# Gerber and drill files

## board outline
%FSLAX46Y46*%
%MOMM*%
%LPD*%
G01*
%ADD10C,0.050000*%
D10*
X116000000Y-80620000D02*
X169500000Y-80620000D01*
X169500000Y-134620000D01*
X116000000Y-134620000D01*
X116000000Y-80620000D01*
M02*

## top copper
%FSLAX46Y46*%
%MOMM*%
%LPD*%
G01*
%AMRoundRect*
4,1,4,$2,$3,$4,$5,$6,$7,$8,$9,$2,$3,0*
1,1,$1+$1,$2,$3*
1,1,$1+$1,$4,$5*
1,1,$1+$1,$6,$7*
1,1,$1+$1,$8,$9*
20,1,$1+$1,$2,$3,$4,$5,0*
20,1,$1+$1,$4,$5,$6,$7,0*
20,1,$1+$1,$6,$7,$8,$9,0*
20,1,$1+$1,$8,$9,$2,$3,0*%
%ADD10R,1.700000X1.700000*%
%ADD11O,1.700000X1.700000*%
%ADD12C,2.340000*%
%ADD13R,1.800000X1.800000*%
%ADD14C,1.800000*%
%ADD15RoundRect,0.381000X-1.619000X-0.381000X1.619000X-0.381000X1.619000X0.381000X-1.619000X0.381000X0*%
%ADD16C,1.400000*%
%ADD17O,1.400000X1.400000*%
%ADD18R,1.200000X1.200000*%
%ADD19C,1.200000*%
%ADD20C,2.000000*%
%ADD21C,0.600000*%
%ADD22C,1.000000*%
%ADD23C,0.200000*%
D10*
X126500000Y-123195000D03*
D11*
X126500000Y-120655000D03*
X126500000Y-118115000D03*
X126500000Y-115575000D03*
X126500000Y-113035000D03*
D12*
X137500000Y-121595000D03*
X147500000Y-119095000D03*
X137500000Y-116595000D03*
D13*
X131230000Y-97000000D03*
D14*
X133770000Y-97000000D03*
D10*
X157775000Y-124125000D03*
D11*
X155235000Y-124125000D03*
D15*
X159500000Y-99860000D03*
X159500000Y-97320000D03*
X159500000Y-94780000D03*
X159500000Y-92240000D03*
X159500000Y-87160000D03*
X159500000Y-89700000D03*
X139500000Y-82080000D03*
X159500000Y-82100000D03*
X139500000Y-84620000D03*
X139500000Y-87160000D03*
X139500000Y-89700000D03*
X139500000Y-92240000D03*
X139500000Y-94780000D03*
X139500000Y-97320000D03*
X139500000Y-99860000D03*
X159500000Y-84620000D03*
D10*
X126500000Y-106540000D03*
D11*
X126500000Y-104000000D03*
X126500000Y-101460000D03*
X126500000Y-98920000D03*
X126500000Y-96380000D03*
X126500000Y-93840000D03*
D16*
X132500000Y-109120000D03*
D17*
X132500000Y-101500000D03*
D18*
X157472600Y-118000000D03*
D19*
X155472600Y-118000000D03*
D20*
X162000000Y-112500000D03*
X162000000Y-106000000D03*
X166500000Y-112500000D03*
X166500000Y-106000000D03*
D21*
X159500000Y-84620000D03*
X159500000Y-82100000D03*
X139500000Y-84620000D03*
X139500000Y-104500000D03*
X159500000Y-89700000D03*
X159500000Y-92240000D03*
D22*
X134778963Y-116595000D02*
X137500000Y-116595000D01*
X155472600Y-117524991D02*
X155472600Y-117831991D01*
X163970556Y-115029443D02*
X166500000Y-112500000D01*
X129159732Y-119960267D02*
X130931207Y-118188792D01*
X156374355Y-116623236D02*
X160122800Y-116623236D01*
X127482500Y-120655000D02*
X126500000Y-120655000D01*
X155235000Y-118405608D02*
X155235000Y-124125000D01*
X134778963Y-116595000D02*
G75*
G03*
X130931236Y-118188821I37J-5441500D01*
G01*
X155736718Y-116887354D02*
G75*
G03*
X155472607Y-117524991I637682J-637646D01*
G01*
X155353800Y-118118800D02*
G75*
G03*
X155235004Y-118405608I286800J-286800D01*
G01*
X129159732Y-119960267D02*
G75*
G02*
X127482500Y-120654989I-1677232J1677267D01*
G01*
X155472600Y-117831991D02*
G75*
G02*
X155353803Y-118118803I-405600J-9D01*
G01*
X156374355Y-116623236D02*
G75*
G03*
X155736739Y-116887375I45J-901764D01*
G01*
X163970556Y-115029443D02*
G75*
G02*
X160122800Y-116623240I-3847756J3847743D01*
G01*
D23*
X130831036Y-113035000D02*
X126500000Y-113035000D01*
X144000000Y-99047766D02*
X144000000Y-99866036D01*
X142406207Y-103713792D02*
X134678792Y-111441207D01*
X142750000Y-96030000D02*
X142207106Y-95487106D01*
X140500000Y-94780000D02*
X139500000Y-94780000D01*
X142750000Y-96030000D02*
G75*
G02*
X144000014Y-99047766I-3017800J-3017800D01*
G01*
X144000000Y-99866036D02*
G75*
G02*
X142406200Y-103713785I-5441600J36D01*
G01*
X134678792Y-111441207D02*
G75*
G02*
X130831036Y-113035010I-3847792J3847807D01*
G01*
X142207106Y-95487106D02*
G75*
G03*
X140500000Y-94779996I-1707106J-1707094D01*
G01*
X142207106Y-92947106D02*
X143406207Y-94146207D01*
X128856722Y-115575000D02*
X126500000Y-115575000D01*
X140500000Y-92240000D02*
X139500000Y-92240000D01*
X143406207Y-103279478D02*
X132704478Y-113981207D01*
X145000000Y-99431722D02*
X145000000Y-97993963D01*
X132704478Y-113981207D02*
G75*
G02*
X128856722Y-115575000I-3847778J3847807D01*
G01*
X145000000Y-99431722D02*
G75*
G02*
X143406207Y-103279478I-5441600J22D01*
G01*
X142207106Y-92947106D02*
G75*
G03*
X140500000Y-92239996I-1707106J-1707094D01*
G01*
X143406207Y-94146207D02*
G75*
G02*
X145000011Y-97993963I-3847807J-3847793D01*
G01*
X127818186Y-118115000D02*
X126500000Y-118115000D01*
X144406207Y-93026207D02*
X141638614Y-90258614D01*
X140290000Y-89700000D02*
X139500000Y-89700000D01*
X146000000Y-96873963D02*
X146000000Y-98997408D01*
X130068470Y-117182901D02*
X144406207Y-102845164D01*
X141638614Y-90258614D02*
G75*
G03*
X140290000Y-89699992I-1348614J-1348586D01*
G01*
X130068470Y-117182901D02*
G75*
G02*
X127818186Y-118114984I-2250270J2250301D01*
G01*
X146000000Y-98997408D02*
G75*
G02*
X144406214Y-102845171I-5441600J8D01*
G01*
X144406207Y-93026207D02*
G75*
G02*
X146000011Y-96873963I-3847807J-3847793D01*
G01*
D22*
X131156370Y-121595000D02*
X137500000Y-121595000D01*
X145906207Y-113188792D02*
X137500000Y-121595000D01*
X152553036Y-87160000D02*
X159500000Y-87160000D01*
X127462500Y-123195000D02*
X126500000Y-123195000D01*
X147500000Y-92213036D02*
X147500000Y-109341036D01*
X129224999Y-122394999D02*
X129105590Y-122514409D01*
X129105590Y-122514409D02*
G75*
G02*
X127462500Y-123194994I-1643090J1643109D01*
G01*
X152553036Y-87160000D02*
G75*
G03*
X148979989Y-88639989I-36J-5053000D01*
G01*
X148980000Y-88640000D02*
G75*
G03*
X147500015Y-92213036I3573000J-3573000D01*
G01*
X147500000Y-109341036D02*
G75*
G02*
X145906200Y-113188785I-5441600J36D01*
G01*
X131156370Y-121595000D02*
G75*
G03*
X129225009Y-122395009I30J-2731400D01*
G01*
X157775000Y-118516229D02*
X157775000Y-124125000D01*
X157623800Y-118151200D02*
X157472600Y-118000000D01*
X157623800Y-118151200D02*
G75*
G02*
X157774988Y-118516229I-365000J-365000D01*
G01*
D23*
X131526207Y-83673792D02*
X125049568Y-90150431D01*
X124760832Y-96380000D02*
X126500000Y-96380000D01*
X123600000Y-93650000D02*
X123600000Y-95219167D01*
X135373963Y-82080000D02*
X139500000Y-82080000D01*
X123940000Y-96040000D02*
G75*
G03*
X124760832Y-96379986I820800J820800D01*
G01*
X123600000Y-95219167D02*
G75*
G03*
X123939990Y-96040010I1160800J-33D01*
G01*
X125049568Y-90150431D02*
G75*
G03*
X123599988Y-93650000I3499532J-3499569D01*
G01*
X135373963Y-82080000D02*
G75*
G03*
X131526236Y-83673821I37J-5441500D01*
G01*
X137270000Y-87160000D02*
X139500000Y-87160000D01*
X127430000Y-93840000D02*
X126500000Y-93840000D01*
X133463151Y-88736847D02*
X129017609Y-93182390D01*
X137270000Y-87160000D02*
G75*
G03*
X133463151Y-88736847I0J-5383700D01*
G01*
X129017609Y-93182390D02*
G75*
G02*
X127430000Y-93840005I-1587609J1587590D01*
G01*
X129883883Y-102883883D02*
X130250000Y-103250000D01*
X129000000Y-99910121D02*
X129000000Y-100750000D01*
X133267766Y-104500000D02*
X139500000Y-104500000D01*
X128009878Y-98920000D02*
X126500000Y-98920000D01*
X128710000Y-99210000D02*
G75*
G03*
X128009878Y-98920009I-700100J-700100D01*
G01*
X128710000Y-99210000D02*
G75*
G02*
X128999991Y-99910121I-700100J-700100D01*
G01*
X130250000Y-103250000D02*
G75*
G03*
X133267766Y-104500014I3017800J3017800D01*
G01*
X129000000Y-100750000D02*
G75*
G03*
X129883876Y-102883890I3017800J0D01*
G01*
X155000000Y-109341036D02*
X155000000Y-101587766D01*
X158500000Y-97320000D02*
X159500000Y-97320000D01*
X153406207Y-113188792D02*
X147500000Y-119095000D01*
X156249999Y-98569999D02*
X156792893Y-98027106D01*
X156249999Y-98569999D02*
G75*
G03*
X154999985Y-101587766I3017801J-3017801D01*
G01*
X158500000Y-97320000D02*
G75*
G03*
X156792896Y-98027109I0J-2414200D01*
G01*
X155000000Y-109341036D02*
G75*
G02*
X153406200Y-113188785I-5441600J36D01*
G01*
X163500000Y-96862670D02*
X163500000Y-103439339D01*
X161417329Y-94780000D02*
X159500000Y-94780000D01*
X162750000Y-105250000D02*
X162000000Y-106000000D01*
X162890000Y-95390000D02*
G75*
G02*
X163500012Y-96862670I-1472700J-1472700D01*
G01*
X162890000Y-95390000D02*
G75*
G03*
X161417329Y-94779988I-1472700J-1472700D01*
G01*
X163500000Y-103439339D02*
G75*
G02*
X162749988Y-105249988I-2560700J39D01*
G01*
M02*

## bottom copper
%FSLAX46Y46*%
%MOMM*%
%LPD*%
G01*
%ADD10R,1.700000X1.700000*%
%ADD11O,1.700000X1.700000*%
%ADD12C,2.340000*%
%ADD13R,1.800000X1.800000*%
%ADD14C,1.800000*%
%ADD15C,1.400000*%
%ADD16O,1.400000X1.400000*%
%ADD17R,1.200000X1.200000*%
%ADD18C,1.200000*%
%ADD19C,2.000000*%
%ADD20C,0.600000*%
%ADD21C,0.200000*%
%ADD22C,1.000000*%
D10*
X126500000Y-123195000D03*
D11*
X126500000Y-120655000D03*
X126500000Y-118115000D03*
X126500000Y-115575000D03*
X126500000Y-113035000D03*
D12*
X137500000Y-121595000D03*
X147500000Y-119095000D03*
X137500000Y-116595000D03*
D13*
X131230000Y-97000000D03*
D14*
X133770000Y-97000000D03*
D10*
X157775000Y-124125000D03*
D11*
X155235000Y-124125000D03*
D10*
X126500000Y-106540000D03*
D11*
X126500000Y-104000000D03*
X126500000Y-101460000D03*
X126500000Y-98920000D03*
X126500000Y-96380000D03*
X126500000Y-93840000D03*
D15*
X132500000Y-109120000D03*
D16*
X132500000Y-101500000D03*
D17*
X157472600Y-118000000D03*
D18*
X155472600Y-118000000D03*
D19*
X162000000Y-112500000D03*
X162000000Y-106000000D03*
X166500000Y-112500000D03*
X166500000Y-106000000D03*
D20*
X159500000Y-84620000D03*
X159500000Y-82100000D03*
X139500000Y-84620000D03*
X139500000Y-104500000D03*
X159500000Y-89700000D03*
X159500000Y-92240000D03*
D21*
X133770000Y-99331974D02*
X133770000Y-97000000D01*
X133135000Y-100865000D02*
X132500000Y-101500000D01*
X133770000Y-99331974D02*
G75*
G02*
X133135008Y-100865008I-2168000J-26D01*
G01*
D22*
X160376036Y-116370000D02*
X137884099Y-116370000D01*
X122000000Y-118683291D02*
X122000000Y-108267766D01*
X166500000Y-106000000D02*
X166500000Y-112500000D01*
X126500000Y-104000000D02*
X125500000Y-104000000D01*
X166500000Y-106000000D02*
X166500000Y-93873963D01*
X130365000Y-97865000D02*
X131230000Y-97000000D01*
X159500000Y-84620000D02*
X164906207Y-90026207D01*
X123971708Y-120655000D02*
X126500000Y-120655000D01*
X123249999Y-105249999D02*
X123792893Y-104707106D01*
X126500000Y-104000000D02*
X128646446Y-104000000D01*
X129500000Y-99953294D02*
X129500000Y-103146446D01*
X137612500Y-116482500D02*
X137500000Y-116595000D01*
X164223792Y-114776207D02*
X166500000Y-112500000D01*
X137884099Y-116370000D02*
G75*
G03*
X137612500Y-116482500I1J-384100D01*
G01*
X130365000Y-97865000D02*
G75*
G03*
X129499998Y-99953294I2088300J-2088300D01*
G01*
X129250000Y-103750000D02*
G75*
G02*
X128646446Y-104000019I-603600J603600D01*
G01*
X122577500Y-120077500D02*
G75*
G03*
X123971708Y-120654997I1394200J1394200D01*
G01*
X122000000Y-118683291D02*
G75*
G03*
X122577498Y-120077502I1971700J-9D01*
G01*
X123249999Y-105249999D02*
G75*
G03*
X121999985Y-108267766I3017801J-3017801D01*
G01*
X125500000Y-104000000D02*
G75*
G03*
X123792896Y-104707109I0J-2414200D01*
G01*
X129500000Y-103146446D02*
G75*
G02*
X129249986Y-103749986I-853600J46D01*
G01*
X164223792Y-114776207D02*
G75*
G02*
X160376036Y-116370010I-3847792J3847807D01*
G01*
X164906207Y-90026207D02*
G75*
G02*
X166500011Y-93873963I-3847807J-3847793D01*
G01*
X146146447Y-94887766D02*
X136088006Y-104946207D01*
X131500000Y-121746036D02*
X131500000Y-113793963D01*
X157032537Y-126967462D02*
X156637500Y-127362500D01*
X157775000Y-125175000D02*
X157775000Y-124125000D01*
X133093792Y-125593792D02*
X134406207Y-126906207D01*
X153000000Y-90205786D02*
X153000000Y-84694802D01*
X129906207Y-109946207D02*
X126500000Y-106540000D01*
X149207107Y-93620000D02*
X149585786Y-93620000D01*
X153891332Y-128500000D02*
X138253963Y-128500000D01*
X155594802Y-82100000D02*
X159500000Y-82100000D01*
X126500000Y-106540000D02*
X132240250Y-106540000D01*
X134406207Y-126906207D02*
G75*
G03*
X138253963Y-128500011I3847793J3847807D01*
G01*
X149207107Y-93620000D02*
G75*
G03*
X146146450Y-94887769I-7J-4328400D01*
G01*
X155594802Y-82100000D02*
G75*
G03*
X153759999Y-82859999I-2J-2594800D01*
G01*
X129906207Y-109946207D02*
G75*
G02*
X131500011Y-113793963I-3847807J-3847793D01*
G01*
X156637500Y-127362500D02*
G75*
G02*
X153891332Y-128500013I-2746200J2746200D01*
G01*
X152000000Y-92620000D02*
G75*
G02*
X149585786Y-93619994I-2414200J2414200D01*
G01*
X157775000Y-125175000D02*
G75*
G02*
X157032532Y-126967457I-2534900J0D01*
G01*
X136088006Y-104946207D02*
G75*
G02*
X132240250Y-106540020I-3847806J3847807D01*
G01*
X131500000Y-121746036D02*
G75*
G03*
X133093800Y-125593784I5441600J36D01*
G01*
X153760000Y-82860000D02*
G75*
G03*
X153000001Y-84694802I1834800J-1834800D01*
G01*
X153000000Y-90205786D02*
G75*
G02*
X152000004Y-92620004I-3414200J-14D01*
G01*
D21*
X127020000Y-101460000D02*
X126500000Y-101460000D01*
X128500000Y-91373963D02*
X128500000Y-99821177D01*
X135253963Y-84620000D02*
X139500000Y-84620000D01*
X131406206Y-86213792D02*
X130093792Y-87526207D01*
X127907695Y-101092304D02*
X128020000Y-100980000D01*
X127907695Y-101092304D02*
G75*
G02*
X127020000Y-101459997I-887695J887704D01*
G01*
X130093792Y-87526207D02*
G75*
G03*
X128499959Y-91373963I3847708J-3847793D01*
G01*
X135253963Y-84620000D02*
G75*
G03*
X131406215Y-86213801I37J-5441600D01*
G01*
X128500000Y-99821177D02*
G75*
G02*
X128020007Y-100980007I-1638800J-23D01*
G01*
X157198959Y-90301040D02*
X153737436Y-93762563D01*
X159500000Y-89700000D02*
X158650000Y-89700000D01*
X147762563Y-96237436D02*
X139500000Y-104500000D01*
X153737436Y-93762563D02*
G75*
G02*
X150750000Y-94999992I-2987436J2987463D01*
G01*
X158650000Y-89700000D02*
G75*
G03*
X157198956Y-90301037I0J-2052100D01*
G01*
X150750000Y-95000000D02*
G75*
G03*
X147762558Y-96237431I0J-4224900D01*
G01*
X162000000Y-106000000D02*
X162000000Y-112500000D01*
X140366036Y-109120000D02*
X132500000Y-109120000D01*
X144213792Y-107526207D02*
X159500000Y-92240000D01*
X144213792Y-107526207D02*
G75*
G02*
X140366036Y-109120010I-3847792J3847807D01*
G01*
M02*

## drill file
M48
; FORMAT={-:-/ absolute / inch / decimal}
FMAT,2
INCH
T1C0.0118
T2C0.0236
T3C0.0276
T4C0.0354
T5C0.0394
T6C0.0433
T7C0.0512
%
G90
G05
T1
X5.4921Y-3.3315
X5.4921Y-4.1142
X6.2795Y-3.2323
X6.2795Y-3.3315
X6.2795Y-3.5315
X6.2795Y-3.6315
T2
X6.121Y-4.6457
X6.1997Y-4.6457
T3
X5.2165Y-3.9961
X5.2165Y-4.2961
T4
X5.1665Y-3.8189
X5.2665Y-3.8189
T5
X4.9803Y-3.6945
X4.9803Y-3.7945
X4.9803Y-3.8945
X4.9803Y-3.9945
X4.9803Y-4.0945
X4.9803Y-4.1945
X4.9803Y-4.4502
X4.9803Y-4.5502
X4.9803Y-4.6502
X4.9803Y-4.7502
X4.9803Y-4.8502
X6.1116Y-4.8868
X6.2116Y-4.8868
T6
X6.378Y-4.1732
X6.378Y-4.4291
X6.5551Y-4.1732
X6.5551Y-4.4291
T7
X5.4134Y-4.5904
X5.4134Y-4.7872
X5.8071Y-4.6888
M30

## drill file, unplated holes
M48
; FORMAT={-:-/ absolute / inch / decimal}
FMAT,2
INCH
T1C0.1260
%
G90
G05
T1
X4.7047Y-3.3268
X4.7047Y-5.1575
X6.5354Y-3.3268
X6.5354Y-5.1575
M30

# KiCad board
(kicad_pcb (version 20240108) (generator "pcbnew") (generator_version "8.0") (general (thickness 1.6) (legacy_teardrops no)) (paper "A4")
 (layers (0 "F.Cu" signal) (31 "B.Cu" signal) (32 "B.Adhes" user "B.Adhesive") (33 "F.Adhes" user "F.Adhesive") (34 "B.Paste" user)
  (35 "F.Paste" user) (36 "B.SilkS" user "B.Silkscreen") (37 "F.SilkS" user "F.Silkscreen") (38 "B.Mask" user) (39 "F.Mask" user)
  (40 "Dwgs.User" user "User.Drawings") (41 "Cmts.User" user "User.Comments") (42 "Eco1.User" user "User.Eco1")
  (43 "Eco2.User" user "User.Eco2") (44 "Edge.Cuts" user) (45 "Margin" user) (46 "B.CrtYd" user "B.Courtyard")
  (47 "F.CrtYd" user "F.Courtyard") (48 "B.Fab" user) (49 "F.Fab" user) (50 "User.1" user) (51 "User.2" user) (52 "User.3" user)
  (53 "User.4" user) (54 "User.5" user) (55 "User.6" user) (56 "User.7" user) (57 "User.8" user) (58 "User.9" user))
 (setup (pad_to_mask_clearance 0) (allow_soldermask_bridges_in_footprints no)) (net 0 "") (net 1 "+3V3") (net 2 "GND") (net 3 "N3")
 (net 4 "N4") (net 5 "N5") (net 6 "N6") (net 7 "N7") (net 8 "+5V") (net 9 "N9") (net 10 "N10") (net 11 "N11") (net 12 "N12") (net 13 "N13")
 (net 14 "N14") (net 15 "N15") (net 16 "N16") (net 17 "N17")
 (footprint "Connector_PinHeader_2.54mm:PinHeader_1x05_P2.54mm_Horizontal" (layer "F.Cu") (at 126.5 123.195 180)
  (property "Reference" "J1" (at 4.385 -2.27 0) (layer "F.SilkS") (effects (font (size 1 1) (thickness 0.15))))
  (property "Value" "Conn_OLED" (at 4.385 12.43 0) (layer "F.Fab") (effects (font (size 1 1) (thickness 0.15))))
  (pad "1" thru_hole rect (at 0 0 180) (size 1.7 1.7) (drill 1) (layers "*.Cu" "*.Mask") (remove_unused_layers no) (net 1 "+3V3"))
  (pad "2" thru_hole oval (at 0 2.54 180) (size 1.7 1.7) (drill 1) (layers "*.Cu" "*.Mask") (remove_unused_layers no) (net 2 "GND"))
  (pad "3" thru_hole oval (at 0 5.08 180) (size 1.7 1.7) (drill 1) (layers "*.Cu" "*.Mask") (remove_unused_layers no) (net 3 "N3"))
  (pad "4" thru_hole oval (at 0 7.62 180) (size 1.7 1.7) (drill 1) (layers "*.Cu" "*.Mask") (remove_unused_layers no) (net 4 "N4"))
  (pad "5" thru_hole oval (at 0 10.16 180) (size 1.7 1.7) (drill 1) (layers "*.Cu" "*.Mask") (remove_unused_layers no) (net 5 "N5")))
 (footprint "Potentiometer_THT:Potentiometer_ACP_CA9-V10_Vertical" (layer "F.Cu") (at 137.5 121.595)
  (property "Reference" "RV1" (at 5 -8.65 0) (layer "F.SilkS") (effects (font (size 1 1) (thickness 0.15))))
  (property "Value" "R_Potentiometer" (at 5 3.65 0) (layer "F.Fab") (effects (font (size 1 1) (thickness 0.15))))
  (pad "1" thru_hole circle (at 0 0) (size 2.34 2.34) (drill 1.3) (layers "*.Cu" "*.Mask") (remove_unused_layers no) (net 1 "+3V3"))
  (pad "2" thru_hole circle (at 10 -2.5) (size 2.34 2.34) (drill 1.3) (layers "*.Cu" "*.Mask") (remove_unused_layers no) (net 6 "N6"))
  (pad "3" thru_hole circle (at 0 -5) (size 2.34 2.34) (drill 1.3) (layers "*.Cu" "*.Mask") (remove_unused_layers no) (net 2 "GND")))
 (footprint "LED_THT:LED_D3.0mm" (layer "F.Cu") (at 131.23 97)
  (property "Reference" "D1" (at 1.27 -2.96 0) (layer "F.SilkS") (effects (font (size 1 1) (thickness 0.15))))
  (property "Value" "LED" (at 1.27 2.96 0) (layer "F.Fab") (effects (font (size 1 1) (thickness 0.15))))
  (pad "1" thru_hole rect (at 0 0) (size 1.8 1.8) (drill 0.9) (layers "*.Cu" "*.Mask") (remove_unused_layers no) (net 2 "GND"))
  (pad "2" thru_hole circle (at 2.54 0) (size 1.8 1.8) (drill 0.9) (layers "*.Cu" "*.Mask") (remove_unused_layers no) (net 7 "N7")))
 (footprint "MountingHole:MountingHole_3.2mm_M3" (layer "F.Cu") (at 119.5 131)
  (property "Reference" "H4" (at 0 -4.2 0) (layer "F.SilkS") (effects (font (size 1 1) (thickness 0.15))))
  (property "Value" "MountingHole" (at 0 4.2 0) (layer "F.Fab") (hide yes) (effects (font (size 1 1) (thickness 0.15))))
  (pad "" np_thru_hole circle (at 0 0) (size 3.2 3.2) (drill 3.2) (layers "*.Cu" "*.Mask")))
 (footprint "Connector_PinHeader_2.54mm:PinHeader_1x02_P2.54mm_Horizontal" (layer "F.Cu") (at 157.775 124.125 -90)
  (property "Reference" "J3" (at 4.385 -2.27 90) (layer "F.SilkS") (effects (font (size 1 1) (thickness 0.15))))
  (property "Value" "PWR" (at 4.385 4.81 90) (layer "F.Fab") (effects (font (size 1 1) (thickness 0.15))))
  (pad "1" thru_hole rect (at 0 0 270) (size 1.7 1.7) (drill 1) (layers "*.Cu" "*.Mask") (remove_unused_layers no) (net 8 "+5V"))
  (pad "2" thru_hole oval (at 0 2.54 270) (size 1.7 1.7) (drill 1) (layers "*.Cu" "*.Mask") (remove_unused_layers no) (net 2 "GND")))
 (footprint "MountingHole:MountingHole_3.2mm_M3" (layer "F.Cu") (at 166 84.5)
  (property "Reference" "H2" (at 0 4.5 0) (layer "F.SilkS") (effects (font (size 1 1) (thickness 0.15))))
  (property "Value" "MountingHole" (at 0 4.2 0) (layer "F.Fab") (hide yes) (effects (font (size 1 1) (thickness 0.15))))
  (pad "" np_thru_hole circle (at 0 0) (size 3.2 3.2) (drill 3.2) (layers "*.Cu" "*.Mask")))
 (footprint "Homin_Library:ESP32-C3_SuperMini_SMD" (layer "F.Cu") (at 149.5 92.08)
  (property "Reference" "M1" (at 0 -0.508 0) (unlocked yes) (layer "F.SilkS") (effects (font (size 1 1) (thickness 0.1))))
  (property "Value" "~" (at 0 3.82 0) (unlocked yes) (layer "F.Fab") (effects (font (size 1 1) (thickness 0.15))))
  (pad "0" smd roundrect (at 10 7.78) (size 4 1.524) (layers "F.Cu" "F.Paste" "F.Mask") (roundrect_rratio 0.25) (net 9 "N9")
   (thermal_bridge_angle 45))
  (pad "1" smd roundrect (at 10 5.24) (size 4 1.524) (layers "F.Cu" "F.Paste" "F.Mask") (roundrect_rratio 0.25) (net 6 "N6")
   (thermal_bridge_angle 45))
  (pad "2" smd roundrect (at 10 2.7) (size 4 1.524) (layers "F.Cu" "F.Paste" "F.Mask") (roundrect_rratio 0.25) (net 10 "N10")
   (thermal_bridge_angle 45))
  (pad "3" smd roundrect (at 10 0.16) (size 4 1.524) (layers "F.Cu" "F.Paste" "F.Mask") (roundrect_rratio 0.25) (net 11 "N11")
   (thermal_bridge_angle 45))
  (pad "3V3" smd roundrect (at 10 -4.92) (size 4 1.524) (layers "F.Cu" "F.Paste" "F.Mask") (roundrect_rratio 0.25) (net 1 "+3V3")
   (thermal_bridge_angle 45))
  (pad "4" smd roundrect (at 10 -2.38) (size 4 1.524) (layers "F.Cu" "F.Paste" "F.Mask") (roundrect_rratio 0.25) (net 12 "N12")
   (thermal_bridge_angle 45))
  (pad "5" smd roundrect (at -10 -10) (size 4 1.524) (layers "F.Cu" "F.Paste" "F.Mask") (roundrect_rratio 0.25) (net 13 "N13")
   (thermal_bridge_angle 45))
  (pad "5V" smd roundrect (at 10 -9.98) (size 4 1.524) (layers "F.Cu" "F.Paste" "F.Mask") (roundrect_rratio 0.25) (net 8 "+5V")
   (thermal_bridge_angle 45))
  (pad "6" smd roundrect (at -10 -7.46) (size 4 1.524) (layers "F.Cu" "F.Paste" "F.Mask") (roundrect_rratio 0.25) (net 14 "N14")
   (thermal_bridge_angle 45))
  (pad "7" smd roundrect (at -10 -4.92) (size 4 1.524) (layers "F.Cu" "F.Paste" "F.Mask") (roundrect_rratio 0.25) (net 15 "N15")
   (thermal_bridge_angle 45))
  (pad "8" smd roundrect (at -10 -2.38) (size 4 1.524) (layers "F.Cu" "F.Paste" "F.Mask") (roundrect_rratio 0.25) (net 3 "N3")
   (thermal_bridge_angle 45))
  (pad "9" smd roundrect (at -10 0.16) (size 4 1.524) (layers "F.Cu" "F.Paste" "F.Mask") (roundrect_rratio 0.25) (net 4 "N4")
   (thermal_bridge_angle 45))
  (pad "10" smd roundrect (at -10 2.7) (size 4 1.524) (layers "F.Cu" "F.Paste" "F.Mask") (roundrect_rratio 0.25) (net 5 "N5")
   (thermal_bridge_angle 45))
  (pad "20" smd roundrect (at -10 5.24) (size 4 1.524) (layers "F.Cu" "F.Paste" "F.Mask") (roundrect_rratio 0.25) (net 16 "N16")
   (thermal_bridge_angle 45))
  (pad "21" smd roundrect (at -10 7.78) (size 4 1.524) (layers "F.Cu" "F.Paste" "F.Mask") (roundrect_rratio 0.25) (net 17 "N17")
   (thermal_bridge_angle 45))
  (pad "G" smd roundrect (at 10 -7.46) (size 4 1.524) (layers "F.Cu" "F.Paste" "F.Mask") (roundrect_rratio 0.25) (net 2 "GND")
   (thermal_bridge_angle 45)))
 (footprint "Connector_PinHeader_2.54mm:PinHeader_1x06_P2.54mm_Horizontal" (layer "F.Cu") (at 126.5 106.54 180)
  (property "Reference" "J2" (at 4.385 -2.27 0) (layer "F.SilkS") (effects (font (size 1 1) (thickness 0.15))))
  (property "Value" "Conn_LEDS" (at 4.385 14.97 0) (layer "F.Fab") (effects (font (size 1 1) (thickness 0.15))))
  (pad "1" thru_hole rect (at 0 0 180) (size 1.7 1.7) (drill 1) (layers "*.Cu" "*.Mask") (remove_unused_layers no) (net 8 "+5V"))
  (pad "2" thru_hole oval (at 0 2.54 180) (size 1.7 1.7) (drill 1) (layers "*.Cu" "*.Mask") (remove_unused_layers no) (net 2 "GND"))
  (pad "3" thru_hole oval (at 0 5.08 180) (size 1.7 1.7) (drill 1) (layers "*.Cu" "*.Mask") (remove_unused_layers no) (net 14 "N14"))
  (pad "4" thru_hole oval (at 0 7.62 180) (size 1.7 1.7) (drill 1) (layers "*.Cu" "*.Mask") (remove_unused_layers no) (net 12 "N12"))
  (pad "5" thru_hole oval (at 0 10.16 180) (size 1.7 1.7) (drill 1) (layers "*.Cu" "*.Mask") (remove_unused_layers no) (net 13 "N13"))
  (pad "6" thru_hole oval (at 0 12.7 180) (size 1.7 1.7) (drill 1) (layers "*.Cu" "*.Mask") (remove_unused_layers no) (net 15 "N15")))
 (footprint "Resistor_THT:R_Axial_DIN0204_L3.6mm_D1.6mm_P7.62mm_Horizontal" (layer "F.Cu") (at 132.5 109.12 90)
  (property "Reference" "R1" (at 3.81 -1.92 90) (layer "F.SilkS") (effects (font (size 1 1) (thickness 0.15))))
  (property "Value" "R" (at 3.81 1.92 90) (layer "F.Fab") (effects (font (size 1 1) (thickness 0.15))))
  (pad "1" thru_hole circle (at 0 0 90) (size 1.4 1.4) (drill 0.7) (layers "*.Cu" "*.Mask") (remove_unused_layers no) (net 11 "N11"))
  (pad "2" thru_hole oval (at 7.62 0 90) (size 1.4 1.4) (drill 0.7) (layers "*.Cu" "*.Mask") (remove_unused_layers no) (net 7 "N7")))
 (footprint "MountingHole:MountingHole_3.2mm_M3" (layer "F.Cu") (at 166 131)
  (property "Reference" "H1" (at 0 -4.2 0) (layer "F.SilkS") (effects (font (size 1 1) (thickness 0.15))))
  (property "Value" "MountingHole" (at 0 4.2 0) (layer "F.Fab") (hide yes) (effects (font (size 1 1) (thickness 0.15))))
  (pad "" np_thru_hole circle (at 0 0) (size 3.2 3.2) (drill 3.2) (layers "*.Cu" "*.Mask")))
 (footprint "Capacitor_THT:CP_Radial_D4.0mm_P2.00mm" (layer "F.Cu") (at 157.4726 118 180)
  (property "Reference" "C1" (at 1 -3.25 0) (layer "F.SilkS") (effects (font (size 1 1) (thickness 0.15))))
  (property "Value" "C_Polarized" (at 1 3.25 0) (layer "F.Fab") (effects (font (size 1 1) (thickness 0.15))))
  (pad "1" thru_hole rect (at 0 0 180) (size 1.2 1.2) (drill 0.6) (layers "*.Cu" "*.Mask") (remove_unused_layers no) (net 8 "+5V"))
  (pad "2" thru_hole circle (at 2 0 180) (size 1.2 1.2) (drill 0.6) (layers "*.Cu" "*.Mask") (remove_unused_layers no) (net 2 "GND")))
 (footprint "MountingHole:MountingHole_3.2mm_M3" (layer "F.Cu") (at 119.5 84.5)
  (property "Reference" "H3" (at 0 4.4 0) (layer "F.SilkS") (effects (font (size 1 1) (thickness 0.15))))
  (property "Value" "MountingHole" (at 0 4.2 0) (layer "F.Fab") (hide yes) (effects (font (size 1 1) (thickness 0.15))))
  (pad "" np_thru_hole circle (at 0 0) (size 3.2 3.2) (drill 3.2) (layers "*.Cu" "*.Mask")))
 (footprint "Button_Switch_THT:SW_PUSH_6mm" (layer "F.Cu") (at 162 112.5 90)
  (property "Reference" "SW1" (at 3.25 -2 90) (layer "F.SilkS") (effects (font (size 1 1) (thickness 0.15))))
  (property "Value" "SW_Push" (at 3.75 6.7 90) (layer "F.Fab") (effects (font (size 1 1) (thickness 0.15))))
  (pad "1" thru_hole circle (at 0 0 180) (size 2 2) (drill 1.1) (layers "*.Cu" "*.Mask") (remove_unused_layers no) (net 10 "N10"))
  (pad "1" thru_hole circle (at 6.5 0 180) (size 2 2) (drill 1.1) (layers "*.Cu" "*.Mask") (remove_unused_layers no) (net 10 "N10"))
  (pad "2" thru_hole circle (at 0 4.5 180) (size 2 2) (drill 1.1) (layers "*.Cu" "*.Mask") (remove_unused_layers no) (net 2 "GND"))
  (pad "2" thru_hole circle (at 6.5 4.5 180) (size 2 2) (drill 1.1) (layers "*.Cu" "*.Mask") (remove_unused_layers no) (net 2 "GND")))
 (gr_rect (start 116 80.62) (end 169.5 134.62) (stroke (width 0.05) (type default)) (fill none) (layer "Edge.Cuts"))
 (segment (start 133.77 99.331974) (end 133.77 97) (width 0.2) (layer "B.Cu") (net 7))
 (segment (start 133.135 100.865) (end 132.5 101.5) (width 0.2) (layer "B.Cu") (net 7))
 (arc (start 133.77 99.331974) (mid 133.604968 100.161641) (end 133.135 100.865) (width 0.2) (layer "B.Cu") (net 7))
 (segment (start 134.778963 116.595) (end 137.5 116.595) (width 1) (layer "F.Cu") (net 2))
 (segment (start 155.4726 117.524991) (end 155.4726 117.831991) (width 1) (layer "F.Cu") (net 2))
 (segment (start 163.970556 115.029443) (end 166.5 112.5) (width 1) (layer "F.Cu") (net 2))
 (segment (start 129.159732 119.960267) (end 130.931207 118.188792) (width 1) (layer "F.Cu") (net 2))
 (segment (start 156.374355 116.623236) (end 160.1228 116.623236) (width 1) (layer "F.Cu") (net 2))
 (segment (start 127.4825 120.655) (end 126.5 120.655) (width 1) (layer "F.Cu") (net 2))
 (segment (start 155.235 118.405608) (end 155.235 124.125) (width 1) (layer "F.Cu") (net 2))
 (via (at 159.5 84.62) (size 0.6) (drill 0.3) (layers "F.Cu" "B.Cu") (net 2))
 (arc (start 134.778963 116.595) (mid 132.696572 117.009213) (end 130.931207 118.188792) (width 1) (layer "F.Cu") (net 2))
 (arc (start 155.736718 116.887354) (mid 155.541242 117.179904) (end 155.4726 117.524991) (width 1) (layer "F.Cu") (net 2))
 (arc (start 155.3538 118.1188) (mid 155.265875 118.250388) (end 155.235 118.405608) (width 1) (layer "F.Cu") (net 2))
 (arc (start 129.159732 119.960267) (mid 128.390211 120.474444) (end 127.4825 120.655) (width 1) (layer "F.Cu") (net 2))
 (arc (start 155.4726 117.831991) (mid 155.441724 117.98721) (end 155.3538 118.1188) (width 1) (layer "F.Cu") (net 2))
 (arc (start 156.374355 116.623236) (mid 156.029268 116.691878) (end 155.736718 116.887354) (width 1) (layer "F.Cu") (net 2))
 (arc (start 163.970556 115.029443) (mid 162.20519 116.209022) (end 160.1228 116.623236) (width 1) (layer "F.Cu") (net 2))
 (segment (start 160.376036 116.37) (end 137.884099 116.37) (width 1) (layer "B.Cu") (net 2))
 (segment (start 122 118.683291) (end 122 108.267766) (width 1) (layer "B.Cu") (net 2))
 (segment (start 166.5 106) (end 166.5 112.5) (width 1) (layer "B.Cu") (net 2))
 (segment (start 126.5 104) (end 125.5 104) (width 1) (layer "B.Cu") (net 2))
 (segment (start 166.5 106) (end 166.5 93.873963) (width 1) (layer "B.Cu") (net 2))
 (segment (start 130.365 97.865) (end 131.23 97) (width 1) (layer "B.Cu") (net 2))
 (segment (start 159.5 84.62) (end 164.906207 90.026207) (width 1) (layer "B.Cu") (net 2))
 (segment (start 123.971708 120.655) (end 126.5 120.655) (width 1) (layer "B.Cu") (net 2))
 (segment (start 123.249999 105.249999) (end 123.792893 104.707106) (width 1) (layer "B.Cu") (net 2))
 (segment (start 126.5 104) (end 128.646446 104) (width 1) (layer "B.Cu") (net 2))
 (segment (start 129.5 99.953294) (end 129.5 103.146446) (width 1) (layer "B.Cu") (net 2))
 (segment (start 137.6125 116.4825) (end 137.5 116.595) (width 1) (layer "B.Cu") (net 2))
 (segment (start 164.223792 114.776207) (end 166.5 112.5) (width 1) (layer "B.Cu") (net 2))
 (arc (start 137.884099 116.37) (mid 137.73711 116.399237) (end 137.6125 116.4825) (width 1) (layer "B.Cu") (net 2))
 (arc (start 130.365 97.865) (mid 129.724806 98.823117) (end 129.5 99.953294) (width 1) (layer "B.Cu") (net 2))
 (arc (start 129.25 103.75) (mid 128.973087 103.935027) (end 128.646446 104) (width 1) (layer "B.Cu") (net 2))
 (arc (start 122.5775 120.0775) (mid 123.217168 120.504912) (end 123.971708 120.655) (width 1) (layer "B.Cu") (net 2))
 (arc (start 122 118.683291) (mid 122.150087 119.437831) (end 122.5775 120.0775) (width 1) (layer "B.Cu") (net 2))
 (arc (start 123.249999 105.249999) (mid 122.324864 106.634562) (end 122 108.267766) (width 1) (layer "B.Cu") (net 2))
 (arc (start 125.5 104) (mid 124.57612 104.18377) (end 123.792893 104.707106) (width 1) (layer "B.Cu") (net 2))
 (arc (start 129.5 103.146446) (mid 129.435027 103.473087) (end 129.25 103.75) (width 1) (layer "B.Cu") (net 2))
 (arc (start 164.223792 114.776207) (mid 162.458426 115.955786) (end 160.376036 116.37) (width 1) (layer "B.Cu") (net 2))
 (arc (start 164.906207 90.026207) (mid 166.085786 91.791572) (end 166.5 93.873963) (width 1) (layer "B.Cu") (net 2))
 (segment (start 130.831036 113.035) (end 126.5 113.035) (width 0.2) (layer "F.Cu") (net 5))
 (segment (start 144 99.047766) (end 144 99.866036) (width 0.2) (layer "F.Cu") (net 5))
 (segment (start 142.406207 103.713792) (end 134.678792 111.441207) (width 0.2) (layer "F.Cu") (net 5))
 (segment (start 142.75 96.03) (end 142.207106 95.487106) (width 0.2) (layer "F.Cu") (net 5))
 (segment (start 140.5 94.78) (end 139.5 94.78) (width 0.2) (layer "F.Cu") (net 5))
 (arc (start 142.75 96.03) (mid 143.675135 97.414562) (end 144 99.047766) (width 0.2) (layer "F.Cu") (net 5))
 (arc (start 144 99.866036) (mid 143.585786 101.948426) (end 142.406207 103.713792) (width 0.2) (layer "F.Cu") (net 5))
 (arc (start 134.678792 111.441207) (mid 132.913426 112.620786) (end 130.831036 113.035) (width 0.2) (layer "F.Cu") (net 5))
 (arc (start 142.207106 95.487106) (mid 141.423879 94.96377) (end 140.5 94.78) (width 0.2) (layer "F.Cu") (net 5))
 (segment (start 142.207106 92.947106) (end 143.406207 94.146207) (width 0.2) (layer "F.Cu") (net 4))
 (segment (start 128.856722 115.575) (end 126.5 115.575) (width 0.2) (layer "F.Cu") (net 4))
 (segment (start 140.5 92.24) (end 139.5 92.24) (width 0.2) (layer "F.Cu") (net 4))
 (segment (start 143.406207 103.279478) (end 132.704478 113.981207) (width 0.2) (layer "F.Cu") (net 4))
 (segment (start 145 99.431722) (end 145 97.993963) (width 0.2) (layer "F.Cu") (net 4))
 (arc (start 132.704478 113.981207) (mid 130.939112 115.160786) (end 128.856722 115.575) (width 0.2) (layer "F.Cu") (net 4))
 (arc (start 145 99.431722) (mid 144.585786 101.514112) (end 143.406207 103.279478) (width 0.2) (layer "F.Cu") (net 4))
 (arc (start 142.207106 92.947106) (mid 141.423879 92.42377) (end 140.5 92.24) (width 0.2) (layer "F.Cu") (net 4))
 (arc (start 143.406207 94.146207) (mid 144.585786 95.911572) (end 145 97.993963) (width 0.2) (layer "F.Cu") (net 4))
 (segment (start 127.818186 118.115) (end 126.5 118.115) (width 0.2) (layer "F.Cu") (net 3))
 (segment (start 144.406207 93.026207) (end 141.638614 90.258614) (width 0.2) (layer "F.Cu") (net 3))
 (segment (start 140.29 89.7) (end 139.5 89.7) (width 0.2) (layer "F.Cu") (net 3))
 (segment (start 146 96.873963) (end 146 98.997408) (width 0.2) (layer "F.Cu") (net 3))
 (segment (start 130.06847 117.182901) (end 144.406207 102.845164) (width 0.2) (layer "F.Cu") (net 3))
 (arc (start 141.638614 90.258614) (mid 141.019864 89.845179) (end 140.29 89.7) (width 0.2) (layer "F.Cu") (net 3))
 (arc (start 130.06847 117.182901) (mid 129.03603 117.872755) (end 127.818186 118.115) (width 0.2) (layer "F.Cu") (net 3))
 (arc (start 146 98.997408) (mid 145.585786 101.079798) (end 144.406207 102.845164) (width 0.2) (layer "F.Cu") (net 3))
 (arc (start 144.406207 93.026207) (mid 145.585786 94.791572) (end 146 96.873963) (width 0.2) (layer "F.Cu") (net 3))
 (segment (start 131.15637 121.595) (end 137.5 121.595) (width 1) (layer "F.Cu") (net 1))
 (segment (start 145.906207 113.188792) (end 137.5 121.595) (width 1) (layer "F.Cu") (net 1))
 (segment (start 152.553036 87.16) (end 159.5 87.16) (width 1) (layer "F.Cu") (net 1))
 (segment (start 127.4625 123.195) (end 126.5 123.195) (width 1) (layer "F.Cu") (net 1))
 (segment (start 147.5 92.213036) (end 147.5 109.341036) (width 1) (layer "F.Cu") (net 1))
 (segment (start 129.224999 122.394999) (end 129.10559 122.514409) (width 1) (layer "F.Cu") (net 1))
 (arc (start 129.10559 122.514409) (mid 128.351733 123.01812) (end 127.4625 123.195) (width 1) (layer "F.Cu") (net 1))
 (arc (start 152.553036 87.16) (mid 150.619322 87.544639) (end 148.98 88.64) (width 1) (layer "F.Cu") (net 1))
 (arc (start 148.98 88.64) (mid 147.884639 90.279322) (end 147.5 92.213036) (width 1) (layer "F.Cu") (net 1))
 (arc (start 147.5 109.341036) (mid 147.085786 111.423426) (end 145.906207 113.188792) (width 1) (layer "F.Cu") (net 1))
 (arc (start 131.15637 121.595) (mid 130.111119 121.802912) (end 129.224999 122.394999) (width 1) (layer "F.Cu") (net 1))
 (segment (start 157.775 118.516229) (end 157.775 124.125) (width 1) (layer "F.Cu") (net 8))
 (segment (start 157.6238 118.1512) (end 157.4726 118) (width 1) (layer "F.Cu") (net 8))
 (via (at 159.5 82.1) (size 0.6) (drill 0.3) (layers "F.Cu" "B.Cu") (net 8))
 (arc (start 157.6238 118.1512) (mid 157.735704 118.318676) (end 157.775 118.516229) (width 1) (layer "F.Cu") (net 8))
 (segment (start 146.146447 94.887766) (end 136.088006 104.946207) (width 1) (layer "B.Cu") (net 8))
 (segment (start 131.5 121.746036) (end 131.5 113.793963) (width 1) (layer "B.Cu") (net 8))
 (segment (start 157.032537 126.967462) (end 156.6375 127.3625) (width 1) (layer "B.Cu") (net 8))
 (segment (start 157.775 125.175) (end 157.775 124.125) (width 1) (layer "B.Cu") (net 8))
 (segment (start 133.093792 125.593792) (end 134.406207 126.906207) (width 1) (layer "B.Cu") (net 8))
 (segment (start 153 90.205786) (end 153 84.694802) (width 1) (layer "B.Cu") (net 8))
 (segment (start 129.906207 109.946207) (end 126.5 106.54) (width 1) (layer "B.Cu") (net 8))
 (segment (start 149.207107 93.62) (end 149.585786 93.62) (width 1) (layer "B.Cu") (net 8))
 (segment (start 153.891332 128.5) (end 138.253963 128.5) (width 1) (layer "B.Cu") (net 8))
 (segment (start 155.594802 82.1) (end 159.5 82.1) (width 1) (layer "B.Cu") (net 8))
 (segment (start 126.5 106.54) (end 132.24025 106.54) (width 1) (layer "B.Cu") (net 8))
 (arc (start 134.406207 126.906207) (mid 136.171572 128.085786) (end 138.253963 128.5) (width 1) (layer "B.Cu") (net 8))
 (arc (start 149.207107 93.62) (mid 147.550689 93.949481) (end 146.146447 94.887766) (width 1) (layer "B.Cu") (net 8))
 (arc (start 155.594802 82.1) (mid 154.601814 82.297517) (end 153.76 82.86) (width 1) (layer "B.Cu") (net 8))
 (arc (start 129.906207 109.946207) (mid 131.085786 111.711572) (end 131.5 113.793963) (width 1) (layer "B.Cu") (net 8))
 (arc (start 156.6375 127.3625) (mid 155.377547 128.204373) (end 153.891332 128.5) (width 1) (layer "B.Cu") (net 8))
 (arc (start 152 92.62) (mid 150.892349 93.360108) (end 149.585786 93.62) (width 1) (layer "B.Cu") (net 8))
 (arc (start 157.775 125.175) (mid 157.58204 126.145073) (end 157.032537 126.967462) (width 1) (layer "B.Cu") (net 8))
 (arc (start 136.088006 104.946207) (mid 134.32264 106.125786) (end 132.24025 106.54) (width 1) (layer "B.Cu") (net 8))
 (arc (start 131.5 121.746036) (mid 131.914213 123.828426) (end 133.093792 125.593792) (width 1) (layer "B.Cu") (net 8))
 (arc (start 153.76 82.86) (mid 153.197517 83.701814) (end 153 84.694802) (width 1) (layer "B.Cu") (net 8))
 (arc (start 153 90.205786) (mid 152.740108 91.512349) (end 152 92.62) (width 1) (layer "B.Cu") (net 8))
 (segment (start 131.526207 83.673792) (end 125.049568 90.150431) (width 0.2) (layer "F.Cu") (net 13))
 (segment (start 124.760832 96.38) (end 126.5 96.38) (width 0.2) (layer "F.Cu") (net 13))
 (segment (start 123.6 93.65) (end 123.6 95.219167) (width 0.2) (layer "F.Cu") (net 13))
 (segment (start 135.373963 82.08) (end 139.5 82.08) (width 0.2) (layer "F.Cu") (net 13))
 (arc (start 123.94 96.04) (mid 124.316601 96.291636) (end 124.760832 96.38) (width 0.2) (layer "F.Cu") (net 13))
 (arc (start 123.6 95.219167) (mid 123.688363 95.663398) (end 123.94 96.04) (width 0.2) (layer "F.Cu") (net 13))
 (arc (start 125.049568 90.150431) (mid 123.97673 91.756046) (end 123.6 93.65) (width 0.2) (layer "F.Cu") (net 13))
 (arc (start 135.373963 82.08) (mid 133.291572 82.494213) (end 131.526207 83.673792) (width 0.2) (layer "F.Cu") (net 13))
 (via (at 139.5 84.62) (size 0.6) (drill 0.3) (layers "F.Cu" "B.Cu") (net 14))
 (segment (start 127.02 101.46) (end 126.5 101.46) (width 0.2) (layer "B.Cu") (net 14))
 (segment (start 128.5 91.373963) (end 128.5 99.821177) (width 0.2) (layer "B.Cu") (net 14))
 (segment (start 135.253963 84.62) (end 139.5 84.62) (width 0.2) (layer "B.Cu") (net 14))
 (segment (start 131.406206 86.213792) (end 130.093792 87.526207) (width 0.2) (layer "B.Cu") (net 14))
 (segment (start 127.907695 101.092304) (end 128.02 100.98) (width 0.2) (layer "B.Cu") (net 14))
 (arc (start 127.907695 101.092304) (mid 127.500417 101.364438) (end 127.02 101.46) (width 0.2) (layer "B.Cu") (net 14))
 (arc (start 130.093792 87.526207) (mid 128.914213 89.291572) (end 128.5 91.373963) (width 0.2) (layer "B.Cu") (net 14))
 (arc (start 135.253963 84.62) (mid 133.171572 85.034213) (end 131.406206 86.213792) (width 0.2) (layer "B.Cu") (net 14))
 (arc (start 128.5 99.821177) (mid 128.375252 100.448327) (end 128.02 100.98) (width 0.2) (layer "B.Cu") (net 14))
 (segment (start 137.27 87.16) (end 139.5 87.16) (width 0.2) (layer "F.Cu") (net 15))
 (segment (start 127.43 93.84) (end 126.5 93.84) (width 0.2) (layer "F.Cu") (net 15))
 (segment (start 133.463151 88.736847) (end 129.017609 93.18239) (width 0.2) (layer "F.Cu") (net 15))
 (arc (start 137.27 87.16) (mid 135.209748 87.569809) (end 133.463151 88.736847) (width 0.2) (layer "F.Cu") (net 15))
 (arc (start 129.017609 93.18239) (mid 128.289207 93.669092) (end 127.43 93.84) (width 0.2) (layer "F.Cu") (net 15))
 (segment (start 129.883883 102.883883) (end 130.25 103.25) (width 0.2) (layer "F.Cu") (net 12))
 (segment (start 129 99.910121) (end 129 100.75) (width 0.2) (layer "F.Cu") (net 12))
 (segment (start 133.267766 104.5) (end 139.5 104.5) (width 0.2) (layer "F.Cu") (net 12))
 (segment (start 128.009878 98.92) (end 126.5 98.92) (width 0.2) (layer "F.Cu") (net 12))
 (via (at 139.5 104.5) (size 0.6) (drill 0.3) (layers "F.Cu" "B.Cu") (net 12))
 (via (at 159.5 89.7) (size 0.6) (drill 0.3) (layers "F.Cu" "B.Cu") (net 12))
 (arc (start 128.71 99.21) (mid 128.388781 98.995368) (end 128.009878 98.92) (width 0.2) (layer "F.Cu") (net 12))
 (arc (start 128.71 99.21) (mid 128.924631 99.531218) (end 129 99.910121) (width 0.2) (layer "F.Cu") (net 12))
 (arc (start 130.25 103.25) (mid 131.634562 104.175135) (end 133.267766 104.5) (width 0.2) (layer "F.Cu") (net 12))
 (arc (start 129 100.75) (mid 129.229713 101.904849) (end 129.883883 102.883883) (width 0.2) (layer "F.Cu") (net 12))
 (segment (start 157.198959 90.30104) (end 153.737436 93.762563) (width 0.2) (layer "B.Cu") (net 12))
 (segment (start 159.5 89.7) (end 158.65 89.7) (width 0.2) (layer "B.Cu") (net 12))
 (segment (start 147.762563 96.237436) (end 139.5 104.5) (width 0.2) (layer "B.Cu") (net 12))
 (arc (start 153.737436 93.762563) (mid 152.366788 94.6784) (end 150.75 95) (width 0.2) (layer "B.Cu") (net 12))
 (arc (start 158.65 89.7) (mid 157.864702 89.856205) (end 157.198959 90.30104) (width 0.2) (layer "B.Cu") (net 12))
 (arc (start 150.75 95) (mid 149.13321 95.321599) (end 147.762563 96.237436) (width 0.2) (layer "B.Cu") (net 12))
 (segment (start 155 109.341036) (end 155 101.587766) (width 0.2) (layer "F.Cu") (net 6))
 (segment (start 158.5 97.32) (end 159.5 97.32) (width 0.2) (layer "F.Cu") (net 6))
 (segment (start 153.406207 113.188792) (end 147.5 119.095) (width 0.2) (layer "F.Cu") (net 6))
 (segment (start 156.249999 98.569999) (end 156.792893 98.027106) (width 0.2) (layer "F.Cu") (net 6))
 (arc (start 156.249999 98.569999) (mid 155.324864 99.954562) (end 155 101.587766) (width 0.2) (layer "F.Cu") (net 6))
 (arc (start 158.5 97.32) (mid 157.57612 97.50377) (end 156.792893 98.027106) (width 0.2) (layer "F.Cu") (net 6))
 (arc (start 155 109.341036) (mid 154.585786 111.423426) (end 153.406207 113.188792) (width 0.2) (layer "F.Cu") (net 6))
 (segment (start 163.5 96.86267) (end 163.5 103.439339) (width 0.2) (layer "F.Cu") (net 10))
 (segment (start 161.417329 94.78) (end 159.5 94.78) (width 0.2) (layer "F.Cu") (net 10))
 (segment (start 162.75 105.25) (end 162 106) (width 0.2) (layer "F.Cu") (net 10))
 (arc (start 162.89 95.39) (mid 163.341466 96.065666) (end 163.5 96.86267) (width 0.2) (layer "F.Cu") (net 10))
 (arc (start 162.89 95.39) (mid 162.214332 94.938533) (end 161.417329 94.78) (width 0.2) (layer "F.Cu") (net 10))
 (arc (start 163.5 103.439339) (mid 163.305081 104.419261) (end 162.75 105.25) (width 0.2) (layer "F.Cu") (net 10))
 (segment (start 162 106) (end 162 112.5) (width 0.2) (layer "B.Cu") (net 10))
 (via (at 159.5 92.24) (size 0.6) (drill 0.3) (layers "F.Cu" "B.Cu") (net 11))
 (segment (start 140.366036 109.12) (end 132.5 109.12) (width 0.2) (layer "B.Cu") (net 11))
 (segment (start 144.213792 107.526207) (end 159.5 92.24) (width 0.2) (layer "B.Cu") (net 11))
 (arc (start 144.213792 107.526207) (mid 142.448426 108.705786) (end 140.366036 109.12) (width 0.2) (layer "B.Cu") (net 11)))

